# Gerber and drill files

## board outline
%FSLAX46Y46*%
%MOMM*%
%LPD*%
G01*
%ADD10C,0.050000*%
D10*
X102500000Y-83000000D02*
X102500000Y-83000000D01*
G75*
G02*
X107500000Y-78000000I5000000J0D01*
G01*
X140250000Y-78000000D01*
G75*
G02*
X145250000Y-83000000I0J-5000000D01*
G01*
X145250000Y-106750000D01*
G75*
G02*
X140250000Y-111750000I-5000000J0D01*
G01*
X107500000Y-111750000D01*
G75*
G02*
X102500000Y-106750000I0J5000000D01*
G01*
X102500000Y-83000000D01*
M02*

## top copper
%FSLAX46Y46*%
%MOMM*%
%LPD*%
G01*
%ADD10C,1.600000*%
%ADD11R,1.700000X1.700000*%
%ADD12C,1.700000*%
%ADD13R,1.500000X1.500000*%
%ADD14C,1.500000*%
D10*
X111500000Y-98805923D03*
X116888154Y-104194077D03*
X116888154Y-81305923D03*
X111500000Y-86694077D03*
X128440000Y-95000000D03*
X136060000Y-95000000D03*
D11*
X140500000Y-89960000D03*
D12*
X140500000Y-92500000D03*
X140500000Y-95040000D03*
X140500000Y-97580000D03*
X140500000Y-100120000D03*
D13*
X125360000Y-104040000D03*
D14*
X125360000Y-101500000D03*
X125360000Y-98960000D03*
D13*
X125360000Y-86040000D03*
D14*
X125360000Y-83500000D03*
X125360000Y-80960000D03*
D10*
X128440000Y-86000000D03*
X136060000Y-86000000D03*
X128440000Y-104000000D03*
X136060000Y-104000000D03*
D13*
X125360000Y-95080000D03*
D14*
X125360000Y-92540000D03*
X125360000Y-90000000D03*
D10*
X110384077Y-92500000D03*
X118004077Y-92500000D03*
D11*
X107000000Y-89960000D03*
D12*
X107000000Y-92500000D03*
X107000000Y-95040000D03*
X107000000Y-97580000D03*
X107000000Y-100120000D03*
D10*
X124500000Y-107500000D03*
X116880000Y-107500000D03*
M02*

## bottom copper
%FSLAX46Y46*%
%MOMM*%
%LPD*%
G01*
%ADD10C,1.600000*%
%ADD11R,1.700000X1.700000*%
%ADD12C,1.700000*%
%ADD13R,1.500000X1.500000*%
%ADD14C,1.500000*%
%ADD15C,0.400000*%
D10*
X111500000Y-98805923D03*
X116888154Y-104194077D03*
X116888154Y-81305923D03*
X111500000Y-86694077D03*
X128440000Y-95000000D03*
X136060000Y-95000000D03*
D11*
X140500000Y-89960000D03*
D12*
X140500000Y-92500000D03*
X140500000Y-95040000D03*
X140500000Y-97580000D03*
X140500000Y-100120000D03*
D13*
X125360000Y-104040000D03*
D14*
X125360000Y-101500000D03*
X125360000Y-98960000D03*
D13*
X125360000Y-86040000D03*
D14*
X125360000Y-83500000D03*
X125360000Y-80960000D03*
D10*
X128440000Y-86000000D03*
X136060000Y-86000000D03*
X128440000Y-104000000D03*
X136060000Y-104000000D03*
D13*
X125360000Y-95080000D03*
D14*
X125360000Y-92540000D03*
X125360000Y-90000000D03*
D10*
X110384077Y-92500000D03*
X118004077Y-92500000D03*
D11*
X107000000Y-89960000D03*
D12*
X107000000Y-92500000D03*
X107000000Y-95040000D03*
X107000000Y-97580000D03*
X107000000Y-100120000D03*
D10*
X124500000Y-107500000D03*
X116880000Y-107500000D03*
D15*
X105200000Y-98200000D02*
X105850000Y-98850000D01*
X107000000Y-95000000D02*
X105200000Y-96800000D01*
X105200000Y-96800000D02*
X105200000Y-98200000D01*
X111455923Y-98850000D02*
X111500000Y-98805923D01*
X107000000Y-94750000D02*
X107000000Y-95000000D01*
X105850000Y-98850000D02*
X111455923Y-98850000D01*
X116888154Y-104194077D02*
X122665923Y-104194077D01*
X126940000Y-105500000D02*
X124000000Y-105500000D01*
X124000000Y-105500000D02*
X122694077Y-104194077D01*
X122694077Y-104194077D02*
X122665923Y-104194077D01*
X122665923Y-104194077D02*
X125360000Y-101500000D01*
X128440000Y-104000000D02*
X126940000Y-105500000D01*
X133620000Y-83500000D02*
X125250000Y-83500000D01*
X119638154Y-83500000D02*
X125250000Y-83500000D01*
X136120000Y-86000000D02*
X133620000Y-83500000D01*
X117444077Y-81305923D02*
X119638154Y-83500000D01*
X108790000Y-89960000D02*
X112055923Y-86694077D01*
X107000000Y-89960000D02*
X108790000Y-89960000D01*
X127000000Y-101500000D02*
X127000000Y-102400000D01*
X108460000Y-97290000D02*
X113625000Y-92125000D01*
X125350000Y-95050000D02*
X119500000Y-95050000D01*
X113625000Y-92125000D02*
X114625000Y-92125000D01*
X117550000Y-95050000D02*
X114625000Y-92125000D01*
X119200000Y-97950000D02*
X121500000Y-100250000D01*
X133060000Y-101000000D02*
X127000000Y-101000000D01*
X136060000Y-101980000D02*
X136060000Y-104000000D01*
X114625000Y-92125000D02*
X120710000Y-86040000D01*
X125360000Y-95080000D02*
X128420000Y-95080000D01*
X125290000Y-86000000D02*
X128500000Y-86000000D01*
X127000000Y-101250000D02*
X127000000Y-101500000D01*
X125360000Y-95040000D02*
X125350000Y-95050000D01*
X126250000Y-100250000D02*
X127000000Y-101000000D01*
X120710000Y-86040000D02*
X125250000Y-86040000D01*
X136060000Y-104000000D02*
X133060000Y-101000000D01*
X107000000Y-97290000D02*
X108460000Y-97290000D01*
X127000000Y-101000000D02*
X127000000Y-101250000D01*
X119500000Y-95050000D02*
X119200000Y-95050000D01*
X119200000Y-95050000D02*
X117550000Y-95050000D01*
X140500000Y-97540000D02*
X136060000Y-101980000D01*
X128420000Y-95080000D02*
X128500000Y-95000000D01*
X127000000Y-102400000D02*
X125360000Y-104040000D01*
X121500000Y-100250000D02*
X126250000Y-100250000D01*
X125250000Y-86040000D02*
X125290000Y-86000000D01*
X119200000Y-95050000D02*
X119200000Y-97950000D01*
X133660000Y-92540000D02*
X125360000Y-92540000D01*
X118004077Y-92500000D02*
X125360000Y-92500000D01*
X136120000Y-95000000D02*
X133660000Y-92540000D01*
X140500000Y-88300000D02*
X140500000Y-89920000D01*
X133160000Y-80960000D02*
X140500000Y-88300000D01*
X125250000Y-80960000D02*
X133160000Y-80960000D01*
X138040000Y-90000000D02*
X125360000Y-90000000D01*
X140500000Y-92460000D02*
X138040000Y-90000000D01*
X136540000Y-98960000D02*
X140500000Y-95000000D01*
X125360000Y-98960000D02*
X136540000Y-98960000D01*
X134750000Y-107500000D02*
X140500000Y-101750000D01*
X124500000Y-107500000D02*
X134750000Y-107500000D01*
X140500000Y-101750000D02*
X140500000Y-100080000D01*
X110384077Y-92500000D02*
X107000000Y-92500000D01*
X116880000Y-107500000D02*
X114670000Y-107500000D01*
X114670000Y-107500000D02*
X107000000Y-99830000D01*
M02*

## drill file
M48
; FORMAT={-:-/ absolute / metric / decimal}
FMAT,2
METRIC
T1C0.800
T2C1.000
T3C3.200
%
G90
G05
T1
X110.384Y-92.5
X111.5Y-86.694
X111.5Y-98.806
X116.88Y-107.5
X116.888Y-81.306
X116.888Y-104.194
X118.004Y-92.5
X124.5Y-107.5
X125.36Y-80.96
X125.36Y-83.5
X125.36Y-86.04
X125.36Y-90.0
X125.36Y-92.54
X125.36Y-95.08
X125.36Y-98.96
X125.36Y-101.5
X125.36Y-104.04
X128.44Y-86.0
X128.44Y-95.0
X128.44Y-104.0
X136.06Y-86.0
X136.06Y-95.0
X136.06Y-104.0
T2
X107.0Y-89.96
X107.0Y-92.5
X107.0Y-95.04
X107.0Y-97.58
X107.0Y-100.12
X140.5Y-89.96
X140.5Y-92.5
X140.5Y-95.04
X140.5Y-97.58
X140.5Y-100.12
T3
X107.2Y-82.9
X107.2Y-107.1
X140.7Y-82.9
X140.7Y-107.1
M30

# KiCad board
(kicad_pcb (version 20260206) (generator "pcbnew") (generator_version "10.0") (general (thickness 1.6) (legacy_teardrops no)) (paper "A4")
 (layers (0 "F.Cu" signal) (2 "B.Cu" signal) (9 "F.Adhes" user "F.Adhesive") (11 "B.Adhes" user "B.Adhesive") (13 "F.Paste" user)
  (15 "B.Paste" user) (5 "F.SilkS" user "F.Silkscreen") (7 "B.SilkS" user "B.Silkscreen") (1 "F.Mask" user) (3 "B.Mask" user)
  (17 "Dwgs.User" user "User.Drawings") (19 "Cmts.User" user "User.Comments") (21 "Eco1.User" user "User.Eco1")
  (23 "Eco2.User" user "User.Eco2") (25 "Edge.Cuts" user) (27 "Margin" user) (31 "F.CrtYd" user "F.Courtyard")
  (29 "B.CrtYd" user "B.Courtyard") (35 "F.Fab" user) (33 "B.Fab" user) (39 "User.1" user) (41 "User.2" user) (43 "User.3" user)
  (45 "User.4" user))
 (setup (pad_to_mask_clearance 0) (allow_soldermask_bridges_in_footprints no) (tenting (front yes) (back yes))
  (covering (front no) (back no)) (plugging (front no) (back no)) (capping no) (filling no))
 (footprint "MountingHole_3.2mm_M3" (layer "F.Cu") (at 140.7 82.9)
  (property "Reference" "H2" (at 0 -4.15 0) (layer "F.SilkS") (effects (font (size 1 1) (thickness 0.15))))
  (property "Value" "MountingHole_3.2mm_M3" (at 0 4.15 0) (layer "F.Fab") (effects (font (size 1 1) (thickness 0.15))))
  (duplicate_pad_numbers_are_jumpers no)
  (pad "" np_thru_hole circle (at 0 0) (size 3.2 3.2) (drill 3.2) (layers "*.Cu" "*.Mask")))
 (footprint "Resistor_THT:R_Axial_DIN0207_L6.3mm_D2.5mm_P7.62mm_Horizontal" (layer "F.Cu") (at 111.5 98.805923 -45)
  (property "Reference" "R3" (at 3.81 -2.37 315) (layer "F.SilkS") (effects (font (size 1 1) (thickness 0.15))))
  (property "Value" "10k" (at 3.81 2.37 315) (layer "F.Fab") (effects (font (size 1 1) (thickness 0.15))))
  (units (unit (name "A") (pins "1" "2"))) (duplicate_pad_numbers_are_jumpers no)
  (pad "1" thru_hole circle (at 0 0 315) (size 1.6 1.6) (drill 0.8) (layers "*.Cu" "*.Mask") (remove_unused_layers no)
   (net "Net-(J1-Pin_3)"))
  (pad "2" thru_hole circle (at 7.62 0 315) (size 1.6 1.6) (drill 0.8) (layers "*.Cu" "*.Mask") (remove_unused_layers no) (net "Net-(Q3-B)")))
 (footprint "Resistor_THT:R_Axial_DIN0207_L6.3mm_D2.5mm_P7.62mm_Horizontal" (layer "F.Cu") (at 116.888154 81.305923 -135)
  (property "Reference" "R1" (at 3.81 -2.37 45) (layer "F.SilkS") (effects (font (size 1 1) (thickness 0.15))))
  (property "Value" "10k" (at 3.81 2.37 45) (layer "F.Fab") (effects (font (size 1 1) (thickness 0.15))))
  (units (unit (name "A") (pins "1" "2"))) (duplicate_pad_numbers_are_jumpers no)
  (pad "1" thru_hole circle (at 0 0 225) (size 1.6 1.6) (drill 0.8) (layers "*.Cu" "*.Mask") (remove_unused_layers no) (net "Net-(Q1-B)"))
  (pad "2" thru_hole circle (at 7.62 0 225) (size 1.6 1.6) (drill 0.8) (layers "*.Cu" "*.Mask") (remove_unused_layers no)
   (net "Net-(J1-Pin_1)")))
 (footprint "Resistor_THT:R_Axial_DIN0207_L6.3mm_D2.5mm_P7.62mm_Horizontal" (layer "F.Cu") (at 128.44 95)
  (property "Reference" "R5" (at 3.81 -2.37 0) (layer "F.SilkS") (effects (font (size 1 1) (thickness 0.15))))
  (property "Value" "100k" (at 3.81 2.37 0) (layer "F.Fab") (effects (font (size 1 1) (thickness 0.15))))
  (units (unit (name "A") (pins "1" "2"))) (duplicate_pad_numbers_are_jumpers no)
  (pad "1" thru_hole circle (at 0 0) (size 1.6 1.6) (drill 0.8) (layers "*.Cu" "*.Mask") (remove_unused_layers no) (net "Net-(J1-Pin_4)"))
  (pad "2" thru_hole circle (at 7.62 0) (size 1.6 1.6) (drill 0.8) (layers "*.Cu" "*.Mask") (remove_unused_layers no) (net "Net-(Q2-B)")))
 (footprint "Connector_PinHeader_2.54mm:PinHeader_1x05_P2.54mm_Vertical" (layer "F.Cu") (at 140.5 89.96)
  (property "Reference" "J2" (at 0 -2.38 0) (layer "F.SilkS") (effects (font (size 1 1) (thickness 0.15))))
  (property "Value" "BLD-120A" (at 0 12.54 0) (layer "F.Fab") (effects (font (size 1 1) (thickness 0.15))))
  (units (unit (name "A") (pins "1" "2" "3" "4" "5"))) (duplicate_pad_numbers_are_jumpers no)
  (pad "1" thru_hole rect (at 0 0) (size 1.7 1.7) (drill 1) (layers "*.Cu" "*.Mask") (remove_unused_layers no) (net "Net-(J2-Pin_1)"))
  (pad "2" thru_hole circle (at 0 2.54) (size 1.7 1.7) (drill 1) (layers "*.Cu" "*.Mask") (remove_unused_layers no) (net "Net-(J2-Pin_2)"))
  (pad "3" thru_hole circle (at 0 5.08) (size 1.7 1.7) (drill 1) (layers "*.Cu" "*.Mask") (remove_unused_layers no) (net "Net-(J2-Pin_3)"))
  (pad "4" thru_hole circle (at 0 7.62) (size 1.7 1.7) (drill 1) (layers "*.Cu" "*.Mask") (remove_unused_layers no) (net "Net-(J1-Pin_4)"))
  (pad "5" thru_hole circle (at 0 10.16) (size 1.7 1.7) (drill 1) (layers "*.Cu" "*.Mask") (remove_unused_layers no) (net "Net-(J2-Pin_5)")))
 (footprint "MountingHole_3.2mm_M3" (layer "F.Cu") (at 140.7 107.1)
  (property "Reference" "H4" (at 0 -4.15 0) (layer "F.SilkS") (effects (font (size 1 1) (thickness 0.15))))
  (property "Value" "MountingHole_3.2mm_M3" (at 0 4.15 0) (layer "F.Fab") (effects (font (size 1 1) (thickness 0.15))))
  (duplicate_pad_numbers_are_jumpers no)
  (pad "" np_thru_hole circle (at 0 0) (size 3.2 3.2) (drill 3.2) (layers "*.Cu" "*.Mask")))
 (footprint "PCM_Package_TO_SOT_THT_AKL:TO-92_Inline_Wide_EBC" (layer "F.Cu") (at 125.36 104.04 90)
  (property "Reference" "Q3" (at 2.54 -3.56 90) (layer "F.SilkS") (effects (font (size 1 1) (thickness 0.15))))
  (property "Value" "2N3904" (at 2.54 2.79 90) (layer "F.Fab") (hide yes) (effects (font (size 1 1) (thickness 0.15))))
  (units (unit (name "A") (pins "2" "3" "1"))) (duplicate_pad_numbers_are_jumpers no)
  (pad "1" thru_hole rect (at 0 0 180) (size 1.5 1.5) (drill 0.8) (layers "*.Cu" "*.Mask") (remove_unused_layers no) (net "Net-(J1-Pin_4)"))
  (pad "2" thru_hole circle (at 2.54 0 180) (size 1.5 1.5) (drill 0.8) (layers "*.Cu" "*.Mask") (remove_unused_layers no) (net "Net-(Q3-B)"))
  (pad "3" thru_hole circle (at 5.08 0 180) (size 1.5 1.5) (drill 0.8) (layers "*.Cu" "*.Mask") (remove_unused_layers no)
   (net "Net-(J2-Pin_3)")))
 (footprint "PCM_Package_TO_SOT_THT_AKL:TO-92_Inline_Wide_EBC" (layer "F.Cu") (at 125.36 86.04 90)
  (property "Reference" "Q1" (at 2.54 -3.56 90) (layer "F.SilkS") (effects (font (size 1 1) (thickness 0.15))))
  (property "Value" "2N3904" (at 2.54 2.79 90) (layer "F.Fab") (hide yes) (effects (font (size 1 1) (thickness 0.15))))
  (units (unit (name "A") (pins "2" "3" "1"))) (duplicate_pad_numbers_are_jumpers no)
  (pad "1" thru_hole rect (at 0 0 180) (size 1.5 1.5) (drill 0.8) (layers "*.Cu" "*.Mask") (remove_unused_layers no) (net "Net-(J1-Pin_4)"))
  (pad "2" thru_hole circle (at 2.54 0 180) (size 1.5 1.5) (drill 0.8) (layers "*.Cu" "*.Mask") (remove_unused_layers no) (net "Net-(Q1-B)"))
  (pad "3" thru_hole circle (at 5.08 0 180) (size 1.5 1.5) (drill 0.8) (layers "*.Cu" "*.Mask") (remove_unused_layers no)
   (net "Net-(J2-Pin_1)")))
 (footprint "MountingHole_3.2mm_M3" (layer "F.Cu") (at 107.2 82.9)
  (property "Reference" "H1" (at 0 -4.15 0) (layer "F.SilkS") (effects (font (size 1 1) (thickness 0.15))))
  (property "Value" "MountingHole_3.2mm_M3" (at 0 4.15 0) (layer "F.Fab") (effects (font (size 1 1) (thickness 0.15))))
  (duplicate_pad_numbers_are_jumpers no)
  (pad "" np_thru_hole circle (at 0 0) (size 3.2 3.2) (drill 3.2) (layers "*.Cu" "*.Mask")))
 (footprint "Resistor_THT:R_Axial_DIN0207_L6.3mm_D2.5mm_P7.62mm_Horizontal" (layer "F.Cu") (at 128.44 86)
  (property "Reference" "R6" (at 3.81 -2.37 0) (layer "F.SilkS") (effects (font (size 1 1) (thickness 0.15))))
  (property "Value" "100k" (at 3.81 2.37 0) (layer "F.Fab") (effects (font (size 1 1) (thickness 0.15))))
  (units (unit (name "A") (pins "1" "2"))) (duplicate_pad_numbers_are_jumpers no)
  (pad "1" thru_hole circle (at 0 0) (size 1.6 1.6) (drill 0.8) (layers "*.Cu" "*.Mask") (remove_unused_layers no) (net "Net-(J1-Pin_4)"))
  (pad "2" thru_hole circle (at 7.62 0) (size 1.6 1.6) (drill 0.8) (layers "*.Cu" "*.Mask") (remove_unused_layers no) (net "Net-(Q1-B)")))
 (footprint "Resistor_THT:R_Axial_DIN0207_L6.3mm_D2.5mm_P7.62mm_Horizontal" (layer "F.Cu") (at 128.44 104)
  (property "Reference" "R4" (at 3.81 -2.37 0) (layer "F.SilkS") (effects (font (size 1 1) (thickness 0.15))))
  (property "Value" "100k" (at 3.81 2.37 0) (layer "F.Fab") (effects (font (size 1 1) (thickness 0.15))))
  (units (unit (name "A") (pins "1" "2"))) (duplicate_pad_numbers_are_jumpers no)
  (pad "1" thru_hole circle (at 0 0) (size 1.6 1.6) (drill 0.8) (layers "*.Cu" "*.Mask") (remove_unused_layers no) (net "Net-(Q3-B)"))
  (pad "2" thru_hole circle (at 7.62 0) (size 1.6 1.6) (drill 0.8) (layers "*.Cu" "*.Mask") (remove_unused_layers no) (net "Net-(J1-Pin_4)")))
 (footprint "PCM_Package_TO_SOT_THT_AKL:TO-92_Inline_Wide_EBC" (layer "F.Cu") (at 125.36 95.08 90)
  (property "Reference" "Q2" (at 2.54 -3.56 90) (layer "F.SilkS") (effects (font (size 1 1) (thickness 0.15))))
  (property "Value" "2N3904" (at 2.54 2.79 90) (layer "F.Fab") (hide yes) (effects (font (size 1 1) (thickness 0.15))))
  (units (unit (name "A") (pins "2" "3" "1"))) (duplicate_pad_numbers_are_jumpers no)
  (pad "1" thru_hole rect (at 0 0 180) (size 1.5 1.5) (drill 0.8) (layers "*.Cu" "*.Mask") (remove_unused_layers no) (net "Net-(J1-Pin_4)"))
  (pad "2" thru_hole circle (at 2.54 0 180) (size 1.5 1.5) (drill 0.8) (layers "*.Cu" "*.Mask") (remove_unused_layers no) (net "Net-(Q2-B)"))
  (pad "3" thru_hole circle (at 5.08 0 180) (size 1.5 1.5) (drill 0.8) (layers "*.Cu" "*.Mask") (remove_unused_layers no)
   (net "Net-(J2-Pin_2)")))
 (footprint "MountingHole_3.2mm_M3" (layer "F.Cu") (at 107.2 107.1)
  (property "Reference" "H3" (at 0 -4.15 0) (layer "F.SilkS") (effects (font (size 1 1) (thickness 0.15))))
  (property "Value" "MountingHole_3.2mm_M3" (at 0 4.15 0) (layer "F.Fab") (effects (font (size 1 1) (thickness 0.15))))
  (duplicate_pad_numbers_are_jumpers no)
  (pad "" np_thru_hole circle (at 0 0) (size 3.2 3.2) (drill 3.2) (layers "*.Cu" "*.Mask")))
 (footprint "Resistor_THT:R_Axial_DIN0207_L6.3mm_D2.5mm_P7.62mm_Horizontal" (layer "F.Cu") (at 110.384077 92.5)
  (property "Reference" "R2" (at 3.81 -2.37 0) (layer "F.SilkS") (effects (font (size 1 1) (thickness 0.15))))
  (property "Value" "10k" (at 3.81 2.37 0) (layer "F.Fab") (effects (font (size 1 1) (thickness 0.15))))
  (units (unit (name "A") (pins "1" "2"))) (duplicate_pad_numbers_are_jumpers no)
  (pad "1" thru_hole circle (at 0 0) (size 1.6 1.6) (drill 0.8) (layers "*.Cu" "*.Mask") (remove_unused_layers no) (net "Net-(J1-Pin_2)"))
  (pad "2" thru_hole circle (at 7.62 0) (size 1.6 1.6) (drill 0.8) (layers "*.Cu" "*.Mask") (remove_unused_layers no) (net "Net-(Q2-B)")))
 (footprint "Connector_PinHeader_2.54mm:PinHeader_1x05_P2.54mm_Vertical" (layer "F.Cu") (at 107 89.96)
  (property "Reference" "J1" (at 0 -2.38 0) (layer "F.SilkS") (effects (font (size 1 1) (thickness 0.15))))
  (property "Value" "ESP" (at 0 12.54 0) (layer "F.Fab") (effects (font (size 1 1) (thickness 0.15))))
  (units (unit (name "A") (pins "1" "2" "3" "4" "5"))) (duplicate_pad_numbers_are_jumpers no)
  (pad "1" thru_hole rect (at 0 0) (size 1.7 1.7) (drill 1) (layers "*.Cu" "*.Mask") (remove_unused_layers no) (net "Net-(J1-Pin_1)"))
  (pad "2" thru_hole circle (at 0 2.54) (size 1.7 1.7) (drill 1) (layers "*.Cu" "*.Mask") (remove_unused_layers no) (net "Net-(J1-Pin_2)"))
  (pad "3" thru_hole circle (at 0 5.08) (size 1.7 1.7) (drill 1) (layers "*.Cu" "*.Mask") (remove_unused_layers no) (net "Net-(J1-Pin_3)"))
  (pad "4" thru_hole circle (at 0 7.62) (size 1.7 1.7) (drill 1) (layers "*.Cu" "*.Mask") (remove_unused_layers no) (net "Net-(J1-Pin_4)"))
  (pad "5" thru_hole circle (at 0 10.16) (size 1.7 1.7) (drill 1) (layers "*.Cu" "*.Mask") (remove_unused_layers no) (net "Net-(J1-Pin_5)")))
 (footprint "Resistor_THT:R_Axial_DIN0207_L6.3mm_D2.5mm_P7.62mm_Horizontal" (layer "B.Cu") (at 124.5 107.5 180)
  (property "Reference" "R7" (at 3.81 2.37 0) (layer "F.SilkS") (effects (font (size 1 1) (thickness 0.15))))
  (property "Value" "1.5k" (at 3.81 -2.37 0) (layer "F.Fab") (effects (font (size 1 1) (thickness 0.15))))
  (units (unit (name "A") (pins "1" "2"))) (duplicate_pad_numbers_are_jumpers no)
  (pad "1" thru_hole circle (at 0 0 180) (size 1.6 1.6) (drill 0.8) (layers "*.Cu" "*.Mask") (remove_unused_layers no)
   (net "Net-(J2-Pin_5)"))
  (pad "2" thru_hole circle (at 7.62 0 180) (size 1.6 1.6) (drill 0.8) (layers "*.Cu" "*.Mask") (remove_unused_layers no)
   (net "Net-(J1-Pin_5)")))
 (gr_rect (start 102.5 78) (end 145.25 111.75) (radius 5) (stroke (width 0.05) (type solid)) (fill no) (layer "Edge.Cuts"))
 (segment (start 105.2 98.2) (end 105.85 98.85) (width 0.4) (layer "B.Cu") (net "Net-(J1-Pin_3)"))
 (segment (start 107 95) (end 105.2 96.8) (width 0.4) (layer "B.Cu") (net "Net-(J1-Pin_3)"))
 (segment (start 105.2 96.8) (end 105.2 98.2) (width 0.4) (layer "B.Cu") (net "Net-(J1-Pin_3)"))
 (segment (start 111.455923 98.85) (end 111.5 98.805923) (width 0.4) (layer "B.Cu") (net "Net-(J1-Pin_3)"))
 (segment (start 107 94.75) (end 107 95) (width 0.4) (layer "B.Cu") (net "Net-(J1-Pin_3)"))
 (segment (start 105.85 98.85) (end 111.455923 98.85) (width 0.4) (layer "B.Cu") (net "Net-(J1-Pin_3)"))
 (segment (start 116.888154 104.194077) (end 122.665923 104.194077) (width 0.4) (layer "B.Cu") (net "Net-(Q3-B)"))
 (segment (start 126.94 105.5) (end 124 105.5) (width 0.4) (layer "B.Cu") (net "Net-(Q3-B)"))
 (segment (start 124 105.5) (end 122.694077 104.194077) (width 0.4) (layer "B.Cu") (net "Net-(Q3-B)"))
 (segment (start 122.694077 104.194077) (end 122.665923 104.194077) (width 0.4) (layer "B.Cu") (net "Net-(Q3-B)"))
 (segment (start 122.665923 104.194077) (end 125.36 101.5) (width 0.4) (layer "B.Cu") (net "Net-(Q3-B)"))
 (segment (start 128.44 104) (end 126.94 105.5) (width 0.4) (layer "B.Cu") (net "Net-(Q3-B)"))
 (segment (start 133.62 83.5) (end 125.25 83.5) (width 0.4) (layer "B.Cu") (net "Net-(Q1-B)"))
 (segment (start 119.638154 83.5) (end 125.25 83.5) (width 0.4) (layer "B.Cu") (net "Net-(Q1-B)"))
 (segment (start 136.12 86) (end 133.62 83.5) (width 0.4) (layer "B.Cu") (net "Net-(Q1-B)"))
 (segment (start 117.444077 81.305923) (end 119.638154 83.5) (width 0.4) (layer "B.Cu") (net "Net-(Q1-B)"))
 (segment (start 108.79 89.96) (end 112.055923 86.694077) (width 0.4) (layer "B.Cu") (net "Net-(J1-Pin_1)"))
 (segment (start 107 89.96) (end 108.79 89.96) (width 0.4) (layer "B.Cu") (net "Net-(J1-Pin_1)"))
 (segment (start 127 101.5) (end 127 102.4) (width 0.4) (layer "B.Cu") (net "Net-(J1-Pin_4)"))
 (segment (start 108.46 97.29) (end 113.625 92.125) (width 0.4) (layer "B.Cu") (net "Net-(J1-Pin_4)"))
 (segment (start 125.35 95.05) (end 119.5 95.05) (width 0.4) (layer "B.Cu") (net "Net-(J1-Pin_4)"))
 (segment (start 113.625 92.125) (end 114.625 92.125) (width 0.4) (layer "B.Cu") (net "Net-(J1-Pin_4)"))
 (segment (start 117.55 95.05) (end 114.625 92.125) (width 0.4) (layer "B.Cu") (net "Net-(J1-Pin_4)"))
 (segment (start 119.2 97.95) (end 121.5 100.25) (width 0.4) (layer "B.Cu") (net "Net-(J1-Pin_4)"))
 (segment (start 133.06 101) (end 127 101) (width 0.4) (layer "B.Cu") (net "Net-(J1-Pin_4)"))
 (segment (start 136.06 101.98) (end 136.06 104) (width 0.4) (layer "B.Cu") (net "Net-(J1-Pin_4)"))
 (segment (start 114.625 92.125) (end 120.71 86.04) (width 0.4) (layer "B.Cu") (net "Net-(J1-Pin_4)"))
 (segment (start 125.36 95.08) (end 128.42 95.08) (width 0.4) (layer "B.Cu") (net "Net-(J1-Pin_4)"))
 (segment (start 125.29 86) (end 128.5 86) (width 0.4) (layer "B.Cu") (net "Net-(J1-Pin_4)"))
 (segment (start 127 101.25) (end 127 101.5) (width 0.4) (layer "B.Cu") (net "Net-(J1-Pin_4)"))
 (segment (start 125.36 95.04) (end 125.35 95.05) (width 0.4) (layer "B.Cu") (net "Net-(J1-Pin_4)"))
 (segment (start 126.25 100.25) (end 127 101) (width 0.4) (layer "B.Cu") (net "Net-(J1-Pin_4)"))
 (segment (start 120.71 86.04) (end 125.25 86.04) (width 0.4) (layer "B.Cu") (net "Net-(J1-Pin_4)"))
 (segment (start 136.06 104) (end 133.06 101) (width 0.4) (layer "B.Cu") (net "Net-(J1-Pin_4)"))
 (segment (start 107 97.29) (end 108.46 97.29) (width 0.4) (layer "B.Cu") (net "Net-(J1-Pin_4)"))
 (segment (start 127 101) (end 127 101.25) (width 0.4) (layer "B.Cu") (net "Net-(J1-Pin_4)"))
 (segment (start 119.5 95.05) (end 119.2 95.05) (width 0.4) (layer "B.Cu") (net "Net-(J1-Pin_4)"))
 (segment (start 119.2 95.05) (end 117.55 95.05) (width 0.4) (layer "B.Cu") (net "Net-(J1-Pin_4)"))
 (segment (start 140.5 97.54) (end 136.06 101.98) (width 0.4) (layer "B.Cu") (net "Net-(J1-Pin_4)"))
 (segment (start 128.42 95.08) (end 128.5 95) (width 0.4) (layer "B.Cu") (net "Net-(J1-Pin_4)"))
 (segment (start 127 102.4) (end 125.36 104.04) (width 0.4) (layer "B.Cu") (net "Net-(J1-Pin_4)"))
 (segment (start 121.5 100.25) (end 126.25 100.25) (width 0.4) (layer "B.Cu") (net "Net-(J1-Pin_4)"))
 (segment (start 125.25 86.04) (end 125.29 86) (width 0.4) (layer "B.Cu") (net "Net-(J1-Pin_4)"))
 (segment (start 119.2 95.05) (end 119.2 97.95) (width 0.4) (layer "B.Cu") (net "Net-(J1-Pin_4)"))
 (segment (start 133.66 92.54) (end 125.36 92.54) (width 0.4) (layer "B.Cu") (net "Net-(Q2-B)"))
 (segment (start 118.004077 92.5) (end 125.36 92.5) (width 0.4) (layer "B.Cu") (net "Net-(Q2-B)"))
 (segment (start 136.12 95) (end 133.66 92.54) (width 0.4) (layer "B.Cu") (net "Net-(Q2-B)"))
 (segment (start 140.5 88.3) (end 140.5 89.92) (width 0.4) (layer "B.Cu") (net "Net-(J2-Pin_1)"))
 (segment (start 133.16 80.96) (end 140.5 88.3) (width 0.4) (layer "B.Cu") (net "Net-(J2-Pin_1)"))
 (segment (start 125.25 80.96) (end 133.16 80.96) (width 0.4) (layer "B.Cu") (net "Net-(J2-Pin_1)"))
 (segment (start 138.04 90) (end 125.36 90) (width 0.4) (layer "B.Cu") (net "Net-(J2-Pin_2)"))
 (segment (start 140.5 92.46) (end 138.04 90) (width 0.4) (layer "B.Cu") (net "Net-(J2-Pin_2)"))
 (segment (start 136.54 98.96) (end 140.5 95) (width 0.4) (layer "B.Cu") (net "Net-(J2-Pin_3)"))
 (segment (start 125.36 98.96) (end 136.54 98.96) (width 0.4) (layer "B.Cu") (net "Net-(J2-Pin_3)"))
 (segment (start 134.75 107.5) (end 140.5 101.75) (width 0.4) (layer "B.Cu") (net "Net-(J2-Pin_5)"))
 (segment (start 124.5 107.5) (end 134.75 107.5) (width 0.4) (layer "B.Cu") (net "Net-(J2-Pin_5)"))
 (segment (start 140.5 101.75) (end 140.5 100.08) (width 0.4) (layer "B.Cu") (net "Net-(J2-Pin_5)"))
 (segment (start 110.384077 92.5) (end 107 92.5) (width 0.4) (layer "B.Cu") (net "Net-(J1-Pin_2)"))
 (segment (start 116.88 107.5) (end 114.67 107.5) (width 0.4) (layer "B.Cu") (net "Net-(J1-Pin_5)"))
 (segment (start 114.67 107.5) (end 107 99.83) (width 0.4) (layer "B.Cu") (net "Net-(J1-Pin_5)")))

